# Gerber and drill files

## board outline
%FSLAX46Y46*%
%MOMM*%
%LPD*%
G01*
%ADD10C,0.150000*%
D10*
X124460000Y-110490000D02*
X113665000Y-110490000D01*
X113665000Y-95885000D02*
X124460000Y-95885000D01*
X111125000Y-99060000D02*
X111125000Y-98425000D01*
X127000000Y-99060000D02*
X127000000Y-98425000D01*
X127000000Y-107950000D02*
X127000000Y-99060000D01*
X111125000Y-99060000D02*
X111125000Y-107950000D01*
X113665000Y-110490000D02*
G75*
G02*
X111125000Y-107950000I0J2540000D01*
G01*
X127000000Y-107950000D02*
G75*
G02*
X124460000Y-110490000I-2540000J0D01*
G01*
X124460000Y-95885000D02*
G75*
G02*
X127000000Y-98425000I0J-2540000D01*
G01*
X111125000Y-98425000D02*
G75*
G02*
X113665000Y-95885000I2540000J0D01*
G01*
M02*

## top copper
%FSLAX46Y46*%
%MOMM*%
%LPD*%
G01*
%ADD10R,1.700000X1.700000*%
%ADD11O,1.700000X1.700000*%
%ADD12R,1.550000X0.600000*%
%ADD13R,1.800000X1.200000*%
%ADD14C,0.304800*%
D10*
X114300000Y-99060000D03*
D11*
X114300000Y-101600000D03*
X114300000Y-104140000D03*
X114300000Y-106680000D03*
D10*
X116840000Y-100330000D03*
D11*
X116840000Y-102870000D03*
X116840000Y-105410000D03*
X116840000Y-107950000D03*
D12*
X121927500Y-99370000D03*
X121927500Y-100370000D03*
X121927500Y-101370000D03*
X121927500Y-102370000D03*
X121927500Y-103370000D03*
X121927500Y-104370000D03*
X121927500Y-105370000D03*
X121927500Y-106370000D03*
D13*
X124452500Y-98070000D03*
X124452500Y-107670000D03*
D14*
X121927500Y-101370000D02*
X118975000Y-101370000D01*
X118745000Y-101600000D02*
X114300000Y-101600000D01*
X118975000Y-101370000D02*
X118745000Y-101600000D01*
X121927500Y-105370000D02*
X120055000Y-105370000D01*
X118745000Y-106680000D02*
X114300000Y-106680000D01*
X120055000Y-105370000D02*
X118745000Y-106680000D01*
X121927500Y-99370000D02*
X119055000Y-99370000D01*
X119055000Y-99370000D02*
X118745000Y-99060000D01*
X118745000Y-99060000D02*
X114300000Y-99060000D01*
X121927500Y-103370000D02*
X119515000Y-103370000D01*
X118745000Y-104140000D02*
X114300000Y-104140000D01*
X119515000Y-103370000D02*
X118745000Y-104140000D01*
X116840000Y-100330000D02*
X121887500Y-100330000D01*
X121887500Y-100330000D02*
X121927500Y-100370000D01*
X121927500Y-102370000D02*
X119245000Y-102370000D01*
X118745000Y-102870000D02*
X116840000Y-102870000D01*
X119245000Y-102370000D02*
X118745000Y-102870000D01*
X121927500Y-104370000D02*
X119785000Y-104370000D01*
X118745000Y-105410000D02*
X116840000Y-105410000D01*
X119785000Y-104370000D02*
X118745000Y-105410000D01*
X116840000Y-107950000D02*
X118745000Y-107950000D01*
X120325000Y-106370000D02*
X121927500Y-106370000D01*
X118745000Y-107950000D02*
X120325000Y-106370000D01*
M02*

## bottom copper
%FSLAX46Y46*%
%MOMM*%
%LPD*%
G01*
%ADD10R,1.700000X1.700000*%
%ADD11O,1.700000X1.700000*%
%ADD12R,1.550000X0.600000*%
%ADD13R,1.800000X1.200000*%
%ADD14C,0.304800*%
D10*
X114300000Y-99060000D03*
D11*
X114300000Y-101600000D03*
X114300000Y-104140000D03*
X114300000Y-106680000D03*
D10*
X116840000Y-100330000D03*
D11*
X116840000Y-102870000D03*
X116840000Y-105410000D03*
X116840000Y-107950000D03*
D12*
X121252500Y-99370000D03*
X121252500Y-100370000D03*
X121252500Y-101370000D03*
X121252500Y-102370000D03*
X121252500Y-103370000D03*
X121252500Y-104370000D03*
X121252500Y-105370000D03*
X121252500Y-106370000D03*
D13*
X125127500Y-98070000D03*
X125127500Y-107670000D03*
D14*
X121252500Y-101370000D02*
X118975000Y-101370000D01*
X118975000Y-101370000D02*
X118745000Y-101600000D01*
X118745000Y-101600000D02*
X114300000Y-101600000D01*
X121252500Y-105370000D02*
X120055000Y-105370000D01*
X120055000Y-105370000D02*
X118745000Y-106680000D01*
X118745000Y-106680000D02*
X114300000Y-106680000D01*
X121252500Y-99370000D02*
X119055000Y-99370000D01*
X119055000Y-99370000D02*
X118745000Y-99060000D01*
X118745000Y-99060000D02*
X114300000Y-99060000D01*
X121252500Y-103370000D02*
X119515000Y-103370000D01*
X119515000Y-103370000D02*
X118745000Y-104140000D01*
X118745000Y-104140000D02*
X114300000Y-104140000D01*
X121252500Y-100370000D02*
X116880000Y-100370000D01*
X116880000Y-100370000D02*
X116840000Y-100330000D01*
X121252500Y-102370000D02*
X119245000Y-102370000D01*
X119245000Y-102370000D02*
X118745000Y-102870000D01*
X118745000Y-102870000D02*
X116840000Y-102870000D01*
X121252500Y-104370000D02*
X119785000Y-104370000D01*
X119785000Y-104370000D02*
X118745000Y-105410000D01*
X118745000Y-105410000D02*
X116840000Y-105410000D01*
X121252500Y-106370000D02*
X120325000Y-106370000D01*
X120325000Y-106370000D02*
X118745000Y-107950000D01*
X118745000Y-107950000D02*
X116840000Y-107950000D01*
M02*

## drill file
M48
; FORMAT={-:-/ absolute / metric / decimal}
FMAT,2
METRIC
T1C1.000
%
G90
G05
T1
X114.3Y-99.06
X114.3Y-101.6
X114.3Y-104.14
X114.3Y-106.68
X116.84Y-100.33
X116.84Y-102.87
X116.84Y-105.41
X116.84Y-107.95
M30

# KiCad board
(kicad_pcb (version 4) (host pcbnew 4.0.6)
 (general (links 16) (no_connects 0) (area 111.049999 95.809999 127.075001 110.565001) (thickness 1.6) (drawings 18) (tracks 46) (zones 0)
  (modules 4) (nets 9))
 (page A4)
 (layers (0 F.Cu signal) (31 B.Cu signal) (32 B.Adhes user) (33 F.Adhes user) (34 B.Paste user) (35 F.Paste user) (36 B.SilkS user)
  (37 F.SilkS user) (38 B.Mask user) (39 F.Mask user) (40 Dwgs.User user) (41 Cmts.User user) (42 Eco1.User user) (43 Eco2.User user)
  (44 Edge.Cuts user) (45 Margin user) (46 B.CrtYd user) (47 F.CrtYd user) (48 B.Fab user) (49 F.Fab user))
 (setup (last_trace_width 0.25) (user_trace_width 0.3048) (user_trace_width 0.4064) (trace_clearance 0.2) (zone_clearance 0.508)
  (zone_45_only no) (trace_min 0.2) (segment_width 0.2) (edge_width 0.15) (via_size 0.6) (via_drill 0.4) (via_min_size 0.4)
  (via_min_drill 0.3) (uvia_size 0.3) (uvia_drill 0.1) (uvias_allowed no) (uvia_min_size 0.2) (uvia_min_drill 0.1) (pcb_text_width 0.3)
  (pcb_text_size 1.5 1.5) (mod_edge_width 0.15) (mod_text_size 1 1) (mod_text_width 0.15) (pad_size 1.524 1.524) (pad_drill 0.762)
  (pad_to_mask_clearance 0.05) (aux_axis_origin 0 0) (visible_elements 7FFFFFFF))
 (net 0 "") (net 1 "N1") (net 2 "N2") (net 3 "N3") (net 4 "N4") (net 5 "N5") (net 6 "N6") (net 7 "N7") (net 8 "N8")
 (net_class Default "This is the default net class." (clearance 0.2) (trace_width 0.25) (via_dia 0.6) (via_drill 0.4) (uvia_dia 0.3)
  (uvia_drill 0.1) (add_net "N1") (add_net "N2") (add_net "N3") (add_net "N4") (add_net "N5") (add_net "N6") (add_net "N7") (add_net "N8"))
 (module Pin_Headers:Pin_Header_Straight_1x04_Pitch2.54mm (layer F.Cu) (at 114.3 99.06)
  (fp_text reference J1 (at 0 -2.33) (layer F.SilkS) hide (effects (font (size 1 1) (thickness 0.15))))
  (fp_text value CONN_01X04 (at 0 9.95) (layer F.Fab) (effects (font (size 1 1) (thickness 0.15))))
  (pad 1 thru_hole rect (at 0 0) (size 1.7 1.7) (drill 1) (layers *.Cu *.Mask) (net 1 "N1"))
  (pad 2 thru_hole oval (at 0 2.54) (size 1.7 1.7) (drill 1) (layers *.Cu *.Mask) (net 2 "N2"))
  (pad 3 thru_hole oval (at 0 5.08) (size 1.7 1.7) (drill 1) (layers *.Cu *.Mask) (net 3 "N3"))
  (pad 4 thru_hole oval (at 0 7.62) (size 1.7 1.7) (drill 1) (layers *.Cu *.Mask) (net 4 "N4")))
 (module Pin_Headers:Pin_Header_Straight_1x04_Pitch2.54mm (layer F.Cu) (at 116.84 100.33)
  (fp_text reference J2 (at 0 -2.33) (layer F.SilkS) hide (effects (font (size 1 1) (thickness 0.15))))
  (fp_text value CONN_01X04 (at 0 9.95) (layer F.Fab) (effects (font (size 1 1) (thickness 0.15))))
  (pad 1 thru_hole rect (at 0 0) (size 1.7 1.7) (drill 1) (layers *.Cu *.Mask) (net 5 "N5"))
  (pad 2 thru_hole oval (at 0 2.54) (size 1.7 1.7) (drill 1) (layers *.Cu *.Mask) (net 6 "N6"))
  (pad 3 thru_hole oval (at 0 5.08) (size 1.7 1.7) (drill 1) (layers *.Cu *.Mask) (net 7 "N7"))
  (pad 4 thru_hole oval (at 0 7.62) (size 1.7 1.7) (drill 1) (layers *.Cu *.Mask) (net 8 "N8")))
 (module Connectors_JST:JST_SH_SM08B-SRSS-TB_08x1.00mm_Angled (layer B.Cu) (at 123.19 102.87 270)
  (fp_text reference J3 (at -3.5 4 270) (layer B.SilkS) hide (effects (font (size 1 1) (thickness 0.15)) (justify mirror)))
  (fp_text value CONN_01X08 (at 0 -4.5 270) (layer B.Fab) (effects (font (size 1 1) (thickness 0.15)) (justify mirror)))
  (pad 1 smd rect (at -3.5 1.9375 270) (size 0.6 1.55) (layers B.Cu B.Paste B.Mask) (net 1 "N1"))
  (pad 2 smd rect (at -2.5 1.9375 270) (size 0.6 1.55) (layers B.Cu B.Paste B.Mask) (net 5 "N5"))
  (pad 3 smd rect (at -1.5 1.9375 270) (size 0.6 1.55) (layers B.Cu B.Paste B.Mask) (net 2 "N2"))
  (pad 4 smd rect (at -0.5 1.9375 270) (size 0.6 1.55) (layers B.Cu B.Paste B.Mask) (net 6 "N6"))
  (pad 5 smd rect (at 0.5 1.9375 270) (size 0.6 1.55) (layers B.Cu B.Paste B.Mask) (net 3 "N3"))
  (pad 6 smd rect (at 1.5 1.9375 270) (size 0.6 1.55) (layers B.Cu B.Paste B.Mask) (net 7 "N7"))
  (pad 7 smd rect (at 2.5 1.9375 270) (size 0.6 1.55) (layers B.Cu B.Paste B.Mask) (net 4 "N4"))
  (pad 8 smd rect (at 3.5 1.9375 270) (size 0.6 1.55) (layers B.Cu B.Paste B.Mask) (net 8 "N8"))
  (pad "" smd rect (at -4.8 -1.9375 270) (size 1.2 1.8) (layers B.Cu B.Paste B.Mask))
  (pad "" smd rect (at 4.8 -1.9375 270) (size 1.2 1.8) (layers B.Cu B.Paste B.Mask)))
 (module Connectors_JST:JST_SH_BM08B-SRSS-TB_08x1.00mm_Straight (layer F.Cu) (at 123.19 102.87 270)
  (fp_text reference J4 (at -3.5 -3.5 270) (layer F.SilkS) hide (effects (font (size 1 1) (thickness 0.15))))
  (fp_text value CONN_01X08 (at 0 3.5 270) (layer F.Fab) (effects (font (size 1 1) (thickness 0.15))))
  (pad 1 smd rect (at -3.5 1.2625 270) (size 0.6 1.55) (layers F.Cu F.Paste F.Mask) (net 1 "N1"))
  (pad 2 smd rect (at -2.5 1.2625 270) (size 0.6 1.55) (layers F.Cu F.Paste F.Mask) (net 5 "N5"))
  (pad 3 smd rect (at -1.5 1.2625 270) (size 0.6 1.55) (layers F.Cu F.Paste F.Mask) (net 2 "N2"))
  (pad 4 smd rect (at -0.5 1.2625 270) (size 0.6 1.55) (layers F.Cu F.Paste F.Mask) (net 6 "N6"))
  (pad 5 smd rect (at 0.5 1.2625 270) (size 0.6 1.55) (layers F.Cu F.Paste F.Mask) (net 3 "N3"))
  (pad 6 smd rect (at 1.5 1.2625 270) (size 0.6 1.55) (layers F.Cu F.Paste F.Mask) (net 7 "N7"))
  (pad 7 smd rect (at 2.5 1.2625 270) (size 0.6 1.55) (layers F.Cu F.Paste F.Mask) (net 4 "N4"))
  (pad 8 smd rect (at 3.5 1.2625 270) (size 0.6 1.55) (layers F.Cu F.Paste F.Mask) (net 8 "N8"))
  (pad "" smd rect (at -4.8 -1.2625 270) (size 1.2 1.8) (layers F.Cu F.Paste F.Mask))
  (pad "" smd rect (at 4.8 -1.2625 270) (size 1.2 1.8) (layers F.Cu F.Paste F.Mask)))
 (gr_line (start 124.46 110.49) (end 113.665 110.49) (angle 90) (layer Edge.Cuts) (width 0.15))
 (gr_line (start 113.665 95.885) (end 124.46 95.885) (angle 90) (layer Edge.Cuts) (width 0.15))
 (gr_line (start 111.125 99.06) (end 111.125 98.425) (angle 90) (layer Edge.Cuts) (width 0.15))
 (gr_line (start 127 99.06) (end 127 98.425) (angle 90) (layer Edge.Cuts) (width 0.15))
 (gr_line (start 127 107.95) (end 127 99.06) (angle 90) (layer Edge.Cuts) (width 0.15))
 (gr_line (start 111.125 99.06) (end 111.125 107.95) (angle 90) (layer Edge.Cuts) (width 0.15))
 (gr_arc (start 113.665 107.95) (end 113.665 110.49) (angle 90) (layer Edge.Cuts) (width 0.15))
 (gr_arc (start 124.46 107.95) (end 127 107.95) (angle 90) (layer Edge.Cuts) (width 0.15))
 (gr_arc (start 124.46 98.425) (end 124.46 95.885) (angle 90) (layer Edge.Cuts) (width 0.15))
 (gr_arc (start 113.665 98.425) (end 111.125 98.425) (angle 90) (layer Edge.Cuts) (width 0.15))
 (segment (start 121.2525 101.37) (end 118.975 101.37) (width 0.3048) (layer B.Cu) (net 2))
 (segment (start 118.975 101.37) (end 118.745 101.6) (width 0.3048) (layer B.Cu) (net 2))
 (segment (start 118.745 101.6) (end 114.3 101.6) (width 0.3048) (layer B.Cu) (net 2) (status 20))
 (segment (start 121.9275 101.37) (end 118.975 101.37) (width 0.3048) (layer F.Cu) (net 2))
 (segment (start 118.745 101.6) (end 114.3 101.6) (width 0.3048) (layer F.Cu) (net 2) (status 20))
 (segment (start 118.975 101.37) (end 118.745 101.6) (width 0.3048) (layer F.Cu) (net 2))
 (segment (start 121.2525 105.37) (end 120.055 105.37) (width 0.3048) (layer B.Cu) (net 4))
 (segment (start 120.055 105.37) (end 118.745 106.68) (width 0.3048) (layer B.Cu) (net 4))
 (segment (start 118.745 106.68) (end 114.3 106.68) (width 0.3048) (layer B.Cu) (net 4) (status 20))
 (segment (start 121.9275 105.37) (end 120.055 105.37) (width 0.3048) (layer F.Cu) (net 4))
 (segment (start 118.745 106.68) (end 114.3 106.68) (width 0.3048) (layer F.Cu) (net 4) (status 20))
 (segment (start 120.055 105.37) (end 118.745 106.68) (width 0.3048) (layer F.Cu) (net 4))
 (segment (start 121.9275 99.37) (end 119.055 99.37) (width 0.3048) (layer F.Cu) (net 1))
 (segment (start 119.055 99.37) (end 118.745 99.06) (width 0.3048) (layer F.Cu) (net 1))
 (segment (start 118.745 99.06) (end 114.3 99.06) (width 0.3048) (layer F.Cu) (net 1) (status 20))
 (segment (start 121.2525 99.37) (end 119.055 99.37) (width 0.3048) (layer B.Cu) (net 1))
 (segment (start 119.055 99.37) (end 118.745 99.06) (width 0.3048) (layer B.Cu) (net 1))
 (segment (start 118.745 99.06) (end 114.3 99.06) (width 0.3048) (layer B.Cu) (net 1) (status 20))
 (segment (start 121.2525 103.37) (end 119.515 103.37) (width 0.3048) (layer B.Cu) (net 3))
 (segment (start 119.515 103.37) (end 118.745 104.14) (width 0.3048) (layer B.Cu) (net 3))
 (segment (start 118.745 104.14) (end 114.3 104.14) (width 0.3048) (layer B.Cu) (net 3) (status 20))
 (segment (start 121.9275 103.37) (end 119.515 103.37) (width 0.3048) (layer F.Cu) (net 3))
 (segment (start 118.745 104.14) (end 114.3 104.14) (width 0.3048) (layer F.Cu) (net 3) (status 20))
 (segment (start 119.515 103.37) (end 118.745 104.14) (width 0.3048) (layer F.Cu) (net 3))
 (segment (start 121.2525 100.37) (end 116.88 100.37) (width 0.3048) (layer B.Cu) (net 5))
 (segment (start 116.88 100.37) (end 116.84 100.33) (width 0.3048) (layer B.Cu) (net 5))
 (segment (start 116.84 100.33) (end 121.8875 100.33) (width 0.3048) (layer F.Cu) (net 5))
 (segment (start 121.8875 100.33) (end 121.9275 100.37) (width 0.3048) (layer F.Cu) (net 5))
 (segment (start 121.2525 102.37) (end 119.245 102.37) (width 0.3048) (layer B.Cu) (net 6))
 (segment (start 119.245 102.37) (end 118.745 102.87) (width 0.3048) (layer B.Cu) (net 6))
 (segment (start 118.745 102.87) (end 116.84 102.87) (width 0.3048) (layer B.Cu) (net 6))
 (segment (start 121.9275 102.37) (end 119.245 102.37) (width 0.3048) (layer F.Cu) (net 6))
 (segment (start 118.745 102.87) (end 116.84 102.87) (width 0.3048) (layer F.Cu) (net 6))
 (segment (start 119.245 102.37) (end 118.745 102.87) (width 0.3048) (layer F.Cu) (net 6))
 (segment (start 121.2525 104.37) (end 119.785 104.37) (width 0.3048) (layer B.Cu) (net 7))
 (segment (start 119.785 104.37) (end 118.745 105.41) (width 0.3048) (layer B.Cu) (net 7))
 (segment (start 118.745 105.41) (end 116.84 105.41) (width 0.3048) (layer B.Cu) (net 7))
 (segment (start 121.9275 104.37) (end 119.785 104.37) (width 0.3048) (layer F.Cu) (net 7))
 (segment (start 118.745 105.41) (end 116.84 105.41) (width 0.3048) (layer F.Cu) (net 7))
 (segment (start 119.785 104.37) (end 118.745 105.41) (width 0.3048) (layer F.Cu) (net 7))
 (segment (start 121.2525 106.37) (end 120.325 106.37) (width 0.3048) (layer B.Cu) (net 8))
 (segment (start 120.325 106.37) (end 118.745 107.95) (width 0.3048) (layer B.Cu) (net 8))
 (segment (start 118.745 107.95) (end 116.84 107.95) (width 0.3048) (layer B.Cu) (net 8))
 (segment (start 116.84 107.95) (end 118.745 107.95) (width 0.3048) (layer F.Cu) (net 8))
 (segment (start 120.325 106.37) (end 121.9275 106.37) (width 0.3048) (layer F.Cu) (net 8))
 (segment (start 118.745 107.95) (end 120.325 106.37) (width 0.3048) (layer F.Cu) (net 8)))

